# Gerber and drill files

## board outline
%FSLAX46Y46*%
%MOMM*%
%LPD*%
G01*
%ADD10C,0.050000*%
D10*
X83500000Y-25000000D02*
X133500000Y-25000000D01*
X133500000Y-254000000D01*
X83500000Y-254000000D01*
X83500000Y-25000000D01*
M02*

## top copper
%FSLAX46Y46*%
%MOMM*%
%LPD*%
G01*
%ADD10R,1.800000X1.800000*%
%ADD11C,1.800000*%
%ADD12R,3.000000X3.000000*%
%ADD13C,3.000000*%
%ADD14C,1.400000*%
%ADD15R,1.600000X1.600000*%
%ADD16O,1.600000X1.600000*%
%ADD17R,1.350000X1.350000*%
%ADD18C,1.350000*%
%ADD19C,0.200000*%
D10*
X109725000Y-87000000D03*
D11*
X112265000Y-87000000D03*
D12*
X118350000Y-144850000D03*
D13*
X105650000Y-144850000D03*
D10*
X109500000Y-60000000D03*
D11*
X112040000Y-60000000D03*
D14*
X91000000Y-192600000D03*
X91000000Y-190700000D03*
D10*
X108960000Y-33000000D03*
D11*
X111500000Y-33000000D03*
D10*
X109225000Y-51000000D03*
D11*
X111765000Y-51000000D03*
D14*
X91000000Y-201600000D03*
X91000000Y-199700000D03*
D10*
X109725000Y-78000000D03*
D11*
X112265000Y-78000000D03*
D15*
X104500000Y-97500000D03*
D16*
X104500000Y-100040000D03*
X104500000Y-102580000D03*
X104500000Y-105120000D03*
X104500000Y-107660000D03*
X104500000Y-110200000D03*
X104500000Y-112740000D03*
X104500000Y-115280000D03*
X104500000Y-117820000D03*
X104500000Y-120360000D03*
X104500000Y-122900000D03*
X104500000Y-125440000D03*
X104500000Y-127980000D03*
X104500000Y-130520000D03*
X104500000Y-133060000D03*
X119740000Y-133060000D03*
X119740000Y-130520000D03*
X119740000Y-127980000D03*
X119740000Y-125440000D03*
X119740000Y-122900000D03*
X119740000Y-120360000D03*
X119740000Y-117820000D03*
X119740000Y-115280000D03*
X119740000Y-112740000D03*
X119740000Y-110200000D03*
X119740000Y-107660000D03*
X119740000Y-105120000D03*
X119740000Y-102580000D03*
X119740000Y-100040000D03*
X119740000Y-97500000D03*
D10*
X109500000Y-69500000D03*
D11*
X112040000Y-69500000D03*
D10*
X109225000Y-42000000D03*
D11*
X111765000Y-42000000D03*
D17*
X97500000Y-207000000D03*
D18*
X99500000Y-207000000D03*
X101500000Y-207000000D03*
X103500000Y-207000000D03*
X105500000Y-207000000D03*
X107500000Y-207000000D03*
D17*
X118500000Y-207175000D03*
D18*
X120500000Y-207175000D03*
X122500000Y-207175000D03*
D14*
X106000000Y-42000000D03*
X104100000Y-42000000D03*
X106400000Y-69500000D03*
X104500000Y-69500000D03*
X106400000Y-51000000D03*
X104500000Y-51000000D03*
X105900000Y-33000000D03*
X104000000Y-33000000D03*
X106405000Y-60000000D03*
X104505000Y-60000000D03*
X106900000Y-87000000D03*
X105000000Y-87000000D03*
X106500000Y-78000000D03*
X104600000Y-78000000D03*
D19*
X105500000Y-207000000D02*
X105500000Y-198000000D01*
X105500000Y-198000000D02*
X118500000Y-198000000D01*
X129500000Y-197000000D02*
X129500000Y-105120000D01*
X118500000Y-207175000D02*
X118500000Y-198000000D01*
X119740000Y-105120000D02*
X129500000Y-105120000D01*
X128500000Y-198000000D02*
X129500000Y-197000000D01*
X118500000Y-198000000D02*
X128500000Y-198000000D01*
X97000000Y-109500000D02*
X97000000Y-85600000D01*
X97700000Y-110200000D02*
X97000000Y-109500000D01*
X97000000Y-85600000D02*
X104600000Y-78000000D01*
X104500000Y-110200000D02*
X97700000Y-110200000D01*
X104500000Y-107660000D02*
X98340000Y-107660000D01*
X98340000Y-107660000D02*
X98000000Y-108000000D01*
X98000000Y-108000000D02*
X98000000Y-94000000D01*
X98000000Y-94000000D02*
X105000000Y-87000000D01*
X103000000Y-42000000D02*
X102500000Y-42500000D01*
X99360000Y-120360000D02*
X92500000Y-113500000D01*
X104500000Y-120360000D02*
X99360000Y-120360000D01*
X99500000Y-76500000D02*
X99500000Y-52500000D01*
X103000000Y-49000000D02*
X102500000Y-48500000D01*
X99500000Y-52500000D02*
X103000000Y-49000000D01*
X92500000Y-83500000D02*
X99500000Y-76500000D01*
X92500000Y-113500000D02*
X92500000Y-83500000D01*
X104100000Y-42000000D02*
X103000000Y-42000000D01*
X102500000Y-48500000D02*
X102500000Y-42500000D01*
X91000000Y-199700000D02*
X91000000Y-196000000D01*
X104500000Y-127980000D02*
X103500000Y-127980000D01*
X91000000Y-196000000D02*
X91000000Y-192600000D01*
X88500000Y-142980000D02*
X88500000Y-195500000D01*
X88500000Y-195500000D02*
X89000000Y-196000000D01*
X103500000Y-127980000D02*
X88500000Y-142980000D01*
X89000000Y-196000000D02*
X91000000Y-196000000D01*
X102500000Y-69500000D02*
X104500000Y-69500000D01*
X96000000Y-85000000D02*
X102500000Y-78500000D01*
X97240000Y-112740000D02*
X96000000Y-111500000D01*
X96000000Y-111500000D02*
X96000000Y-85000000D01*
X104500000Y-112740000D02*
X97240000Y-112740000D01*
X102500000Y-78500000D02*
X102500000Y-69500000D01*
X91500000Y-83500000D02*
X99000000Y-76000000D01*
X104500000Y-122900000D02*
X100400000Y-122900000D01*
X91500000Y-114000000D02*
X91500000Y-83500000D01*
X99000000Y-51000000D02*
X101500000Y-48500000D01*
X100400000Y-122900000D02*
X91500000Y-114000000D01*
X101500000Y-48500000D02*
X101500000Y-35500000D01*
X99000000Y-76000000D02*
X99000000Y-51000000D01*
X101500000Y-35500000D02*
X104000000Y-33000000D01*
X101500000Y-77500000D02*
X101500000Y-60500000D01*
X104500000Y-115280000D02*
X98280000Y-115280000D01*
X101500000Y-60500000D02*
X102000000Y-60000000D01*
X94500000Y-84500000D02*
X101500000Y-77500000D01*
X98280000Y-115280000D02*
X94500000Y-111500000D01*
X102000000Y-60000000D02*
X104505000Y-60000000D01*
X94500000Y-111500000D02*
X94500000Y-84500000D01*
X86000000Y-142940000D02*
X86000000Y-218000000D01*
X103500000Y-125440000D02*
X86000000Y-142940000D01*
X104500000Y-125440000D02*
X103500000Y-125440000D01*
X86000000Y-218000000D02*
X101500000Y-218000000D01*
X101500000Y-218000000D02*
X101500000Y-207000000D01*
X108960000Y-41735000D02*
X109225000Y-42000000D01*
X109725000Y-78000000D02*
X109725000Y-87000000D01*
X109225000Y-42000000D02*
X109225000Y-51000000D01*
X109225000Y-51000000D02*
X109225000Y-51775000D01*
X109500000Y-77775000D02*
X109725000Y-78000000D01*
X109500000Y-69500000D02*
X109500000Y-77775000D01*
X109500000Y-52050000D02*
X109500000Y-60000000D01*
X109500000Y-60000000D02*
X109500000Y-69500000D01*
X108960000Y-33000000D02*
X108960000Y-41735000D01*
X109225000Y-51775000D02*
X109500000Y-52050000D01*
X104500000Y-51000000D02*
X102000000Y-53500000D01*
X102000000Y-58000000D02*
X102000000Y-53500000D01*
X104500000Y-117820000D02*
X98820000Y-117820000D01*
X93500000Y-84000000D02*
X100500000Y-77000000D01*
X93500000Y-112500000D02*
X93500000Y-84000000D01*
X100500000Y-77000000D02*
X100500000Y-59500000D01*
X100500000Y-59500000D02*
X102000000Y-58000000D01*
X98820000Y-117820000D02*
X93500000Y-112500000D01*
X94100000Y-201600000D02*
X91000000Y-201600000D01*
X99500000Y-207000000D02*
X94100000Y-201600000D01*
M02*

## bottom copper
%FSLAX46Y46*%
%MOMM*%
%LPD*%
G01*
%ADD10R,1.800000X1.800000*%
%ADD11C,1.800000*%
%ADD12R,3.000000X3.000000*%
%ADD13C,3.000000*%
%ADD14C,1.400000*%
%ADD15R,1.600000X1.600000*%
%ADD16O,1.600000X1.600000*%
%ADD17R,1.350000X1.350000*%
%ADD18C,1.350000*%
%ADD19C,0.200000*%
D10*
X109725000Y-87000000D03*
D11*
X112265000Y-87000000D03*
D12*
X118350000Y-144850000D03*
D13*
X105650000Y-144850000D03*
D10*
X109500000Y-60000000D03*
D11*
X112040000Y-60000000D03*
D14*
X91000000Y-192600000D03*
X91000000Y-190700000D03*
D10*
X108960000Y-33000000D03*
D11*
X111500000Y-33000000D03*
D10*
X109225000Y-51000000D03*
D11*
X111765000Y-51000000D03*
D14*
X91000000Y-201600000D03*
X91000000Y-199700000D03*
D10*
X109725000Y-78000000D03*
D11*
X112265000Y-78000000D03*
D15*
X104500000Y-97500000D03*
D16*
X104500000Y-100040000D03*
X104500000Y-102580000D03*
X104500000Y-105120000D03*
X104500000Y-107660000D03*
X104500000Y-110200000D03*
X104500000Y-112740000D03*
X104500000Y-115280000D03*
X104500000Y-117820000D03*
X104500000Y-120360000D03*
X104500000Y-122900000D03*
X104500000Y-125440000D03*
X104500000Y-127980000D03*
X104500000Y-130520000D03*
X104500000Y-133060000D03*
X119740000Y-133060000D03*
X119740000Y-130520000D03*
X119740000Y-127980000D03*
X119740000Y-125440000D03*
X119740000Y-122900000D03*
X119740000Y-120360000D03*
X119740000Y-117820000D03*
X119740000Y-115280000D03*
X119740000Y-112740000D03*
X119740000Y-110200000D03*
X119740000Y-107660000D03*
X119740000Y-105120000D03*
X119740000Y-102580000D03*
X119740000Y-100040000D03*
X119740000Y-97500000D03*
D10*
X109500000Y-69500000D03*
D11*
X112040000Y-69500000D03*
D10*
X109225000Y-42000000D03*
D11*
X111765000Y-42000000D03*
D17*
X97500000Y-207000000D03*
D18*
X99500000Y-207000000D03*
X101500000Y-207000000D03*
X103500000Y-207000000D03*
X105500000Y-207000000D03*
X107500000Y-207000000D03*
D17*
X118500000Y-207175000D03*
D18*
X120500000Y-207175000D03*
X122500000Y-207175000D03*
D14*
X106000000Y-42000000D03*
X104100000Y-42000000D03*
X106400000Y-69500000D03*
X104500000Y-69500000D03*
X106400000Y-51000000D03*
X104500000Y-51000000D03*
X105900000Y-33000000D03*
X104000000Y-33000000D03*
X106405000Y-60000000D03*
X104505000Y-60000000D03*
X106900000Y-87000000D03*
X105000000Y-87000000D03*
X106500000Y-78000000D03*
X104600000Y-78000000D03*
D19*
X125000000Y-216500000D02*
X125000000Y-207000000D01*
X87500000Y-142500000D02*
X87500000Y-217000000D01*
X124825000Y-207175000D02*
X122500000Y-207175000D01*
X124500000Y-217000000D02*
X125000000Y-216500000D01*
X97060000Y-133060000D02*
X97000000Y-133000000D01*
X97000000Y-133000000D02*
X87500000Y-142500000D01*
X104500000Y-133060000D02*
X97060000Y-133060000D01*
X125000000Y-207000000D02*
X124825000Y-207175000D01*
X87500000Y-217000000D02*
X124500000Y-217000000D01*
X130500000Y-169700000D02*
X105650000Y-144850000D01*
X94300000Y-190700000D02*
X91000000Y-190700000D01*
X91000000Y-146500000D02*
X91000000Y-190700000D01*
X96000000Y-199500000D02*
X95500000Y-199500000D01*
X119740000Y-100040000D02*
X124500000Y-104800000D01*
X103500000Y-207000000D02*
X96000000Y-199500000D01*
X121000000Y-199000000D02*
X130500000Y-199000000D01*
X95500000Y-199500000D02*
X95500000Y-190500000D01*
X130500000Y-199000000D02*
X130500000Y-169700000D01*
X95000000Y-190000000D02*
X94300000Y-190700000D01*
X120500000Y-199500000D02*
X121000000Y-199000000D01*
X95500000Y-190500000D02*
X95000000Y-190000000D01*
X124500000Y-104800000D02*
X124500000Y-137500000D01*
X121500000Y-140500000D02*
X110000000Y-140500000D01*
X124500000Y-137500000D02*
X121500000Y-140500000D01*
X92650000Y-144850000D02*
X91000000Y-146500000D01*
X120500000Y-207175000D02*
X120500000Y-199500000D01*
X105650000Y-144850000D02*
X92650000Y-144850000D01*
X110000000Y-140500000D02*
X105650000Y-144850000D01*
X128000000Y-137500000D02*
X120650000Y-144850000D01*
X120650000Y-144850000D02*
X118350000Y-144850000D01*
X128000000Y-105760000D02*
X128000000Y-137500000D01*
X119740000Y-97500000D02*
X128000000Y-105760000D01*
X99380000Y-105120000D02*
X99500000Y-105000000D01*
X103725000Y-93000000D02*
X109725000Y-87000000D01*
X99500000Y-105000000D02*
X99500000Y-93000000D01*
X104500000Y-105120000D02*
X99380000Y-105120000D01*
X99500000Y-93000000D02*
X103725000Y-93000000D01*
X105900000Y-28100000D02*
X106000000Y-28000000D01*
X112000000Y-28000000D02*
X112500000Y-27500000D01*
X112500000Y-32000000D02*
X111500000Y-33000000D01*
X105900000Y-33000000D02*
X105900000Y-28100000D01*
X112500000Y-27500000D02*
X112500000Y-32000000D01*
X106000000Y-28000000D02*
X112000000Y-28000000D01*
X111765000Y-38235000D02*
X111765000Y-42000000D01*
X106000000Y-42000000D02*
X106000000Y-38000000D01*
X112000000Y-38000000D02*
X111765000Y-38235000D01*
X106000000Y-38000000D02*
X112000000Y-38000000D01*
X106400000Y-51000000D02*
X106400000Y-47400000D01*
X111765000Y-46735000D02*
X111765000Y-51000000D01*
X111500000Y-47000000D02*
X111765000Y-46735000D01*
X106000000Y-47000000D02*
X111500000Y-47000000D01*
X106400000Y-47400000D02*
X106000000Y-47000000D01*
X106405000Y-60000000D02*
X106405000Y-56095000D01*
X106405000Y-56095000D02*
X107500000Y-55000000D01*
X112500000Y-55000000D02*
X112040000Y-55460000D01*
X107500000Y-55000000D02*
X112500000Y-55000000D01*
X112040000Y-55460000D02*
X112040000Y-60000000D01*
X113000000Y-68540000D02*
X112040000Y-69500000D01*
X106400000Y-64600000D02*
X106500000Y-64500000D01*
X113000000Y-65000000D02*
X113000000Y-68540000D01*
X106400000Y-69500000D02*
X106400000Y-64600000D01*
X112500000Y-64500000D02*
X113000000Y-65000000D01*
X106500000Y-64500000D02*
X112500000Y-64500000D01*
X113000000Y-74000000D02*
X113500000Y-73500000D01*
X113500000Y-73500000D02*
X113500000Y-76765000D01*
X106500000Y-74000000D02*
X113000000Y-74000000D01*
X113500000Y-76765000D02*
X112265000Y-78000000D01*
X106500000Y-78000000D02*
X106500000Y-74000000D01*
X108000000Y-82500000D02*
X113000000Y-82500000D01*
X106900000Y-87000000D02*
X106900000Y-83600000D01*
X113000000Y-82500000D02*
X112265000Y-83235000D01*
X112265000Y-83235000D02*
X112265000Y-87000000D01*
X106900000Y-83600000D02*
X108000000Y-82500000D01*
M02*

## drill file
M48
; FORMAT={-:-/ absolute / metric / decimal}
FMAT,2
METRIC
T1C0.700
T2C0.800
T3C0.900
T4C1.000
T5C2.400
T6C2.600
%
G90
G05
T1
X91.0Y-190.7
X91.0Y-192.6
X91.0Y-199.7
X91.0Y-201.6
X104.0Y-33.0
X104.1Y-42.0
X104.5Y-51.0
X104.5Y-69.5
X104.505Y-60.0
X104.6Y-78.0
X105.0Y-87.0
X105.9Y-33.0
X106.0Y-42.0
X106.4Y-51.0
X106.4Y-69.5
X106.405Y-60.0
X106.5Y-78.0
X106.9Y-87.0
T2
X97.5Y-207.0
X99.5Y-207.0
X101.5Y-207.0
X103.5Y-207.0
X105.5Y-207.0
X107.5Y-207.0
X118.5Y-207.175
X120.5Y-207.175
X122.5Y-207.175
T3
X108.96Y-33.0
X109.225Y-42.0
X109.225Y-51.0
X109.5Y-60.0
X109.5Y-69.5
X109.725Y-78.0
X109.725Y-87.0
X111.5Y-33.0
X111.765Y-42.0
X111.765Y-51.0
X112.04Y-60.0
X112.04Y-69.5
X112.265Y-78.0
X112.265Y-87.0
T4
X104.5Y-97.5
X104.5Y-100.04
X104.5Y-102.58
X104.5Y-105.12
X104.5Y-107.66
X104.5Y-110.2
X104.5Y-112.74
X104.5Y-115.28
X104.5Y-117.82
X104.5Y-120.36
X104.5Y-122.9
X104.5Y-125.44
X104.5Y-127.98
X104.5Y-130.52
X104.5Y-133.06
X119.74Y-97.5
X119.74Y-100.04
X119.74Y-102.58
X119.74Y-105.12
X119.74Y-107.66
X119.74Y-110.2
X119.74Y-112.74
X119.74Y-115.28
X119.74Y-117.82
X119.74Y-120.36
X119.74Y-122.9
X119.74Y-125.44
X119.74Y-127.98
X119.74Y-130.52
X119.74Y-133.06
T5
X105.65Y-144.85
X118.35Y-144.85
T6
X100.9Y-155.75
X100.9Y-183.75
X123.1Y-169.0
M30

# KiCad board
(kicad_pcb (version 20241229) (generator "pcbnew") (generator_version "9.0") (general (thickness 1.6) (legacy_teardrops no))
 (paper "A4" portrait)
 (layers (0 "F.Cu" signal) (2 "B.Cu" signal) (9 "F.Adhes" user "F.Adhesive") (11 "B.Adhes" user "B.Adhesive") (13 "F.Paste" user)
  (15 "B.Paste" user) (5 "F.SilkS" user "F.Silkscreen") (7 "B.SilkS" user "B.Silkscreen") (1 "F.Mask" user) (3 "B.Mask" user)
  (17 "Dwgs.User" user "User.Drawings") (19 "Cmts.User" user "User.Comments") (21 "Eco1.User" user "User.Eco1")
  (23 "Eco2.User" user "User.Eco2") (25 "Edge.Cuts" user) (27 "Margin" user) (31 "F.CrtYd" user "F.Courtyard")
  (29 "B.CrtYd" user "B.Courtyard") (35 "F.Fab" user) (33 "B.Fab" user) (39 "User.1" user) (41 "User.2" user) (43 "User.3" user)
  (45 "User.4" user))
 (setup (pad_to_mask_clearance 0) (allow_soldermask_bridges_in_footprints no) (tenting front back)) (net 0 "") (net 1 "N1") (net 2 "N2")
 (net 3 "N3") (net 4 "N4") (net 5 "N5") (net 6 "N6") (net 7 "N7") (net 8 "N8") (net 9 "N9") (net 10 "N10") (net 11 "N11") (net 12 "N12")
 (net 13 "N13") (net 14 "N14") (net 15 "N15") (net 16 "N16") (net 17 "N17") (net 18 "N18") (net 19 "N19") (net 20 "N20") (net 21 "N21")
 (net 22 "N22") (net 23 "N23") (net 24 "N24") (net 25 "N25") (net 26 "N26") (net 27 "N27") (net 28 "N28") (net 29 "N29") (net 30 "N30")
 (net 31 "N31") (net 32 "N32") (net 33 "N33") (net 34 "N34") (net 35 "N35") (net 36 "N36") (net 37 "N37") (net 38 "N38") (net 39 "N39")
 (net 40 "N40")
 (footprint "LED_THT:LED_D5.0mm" (layer "F.Cu") (at 109.725 87)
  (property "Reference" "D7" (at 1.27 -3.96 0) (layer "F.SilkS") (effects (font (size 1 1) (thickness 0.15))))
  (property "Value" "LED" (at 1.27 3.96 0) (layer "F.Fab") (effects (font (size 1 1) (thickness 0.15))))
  (pad "1" thru_hole rect (at 0 0) (size 1.8 1.8) (drill 0.9) (layers "*.Cu" "*.Mask") (remove_unused_layers no) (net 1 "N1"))
  (pad "2" thru_hole circle (at 2.54 0) (size 1.8 1.8) (drill 0.9) (layers "*.Cu" "*.Mask") (remove_unused_layers no) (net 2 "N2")))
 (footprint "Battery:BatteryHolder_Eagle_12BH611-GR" (layer "F.Cu") (at 118.35 144.85 90)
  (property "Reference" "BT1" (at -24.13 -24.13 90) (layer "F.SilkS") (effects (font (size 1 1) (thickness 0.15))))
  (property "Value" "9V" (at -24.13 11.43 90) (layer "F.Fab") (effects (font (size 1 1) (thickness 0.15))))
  (pad "" np_thru_hole circle (at -38.9 -17.45 90) (size 2.6 2.6) (drill 2.6) (layers "*.Cu" "*.Mask"))
  (pad "" np_thru_hole circle (at -24.15 4.75 90) (size 2.6 2.6) (drill 2.6) (layers "*.Cu" "*.Mask"))
  (pad "" np_thru_hole circle (at -10.9 -17.45 90) (size 2.6 2.6) (drill 2.6) (layers "*.Cu" "*.Mask"))
  (pad "1" thru_hole rect (at 0 0 90) (size 3 3) (drill 2.4) (layers "*.Cu" "*.Mask") (remove_unused_layers no) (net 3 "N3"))
  (pad "2" thru_hole circle (at 0 -12.7 90) (size 3 3) (drill 2.4) (layers "*.Cu" "*.Mask") (remove_unused_layers no) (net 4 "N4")))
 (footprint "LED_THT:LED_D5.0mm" (layer "F.Cu") (at 109.5 60)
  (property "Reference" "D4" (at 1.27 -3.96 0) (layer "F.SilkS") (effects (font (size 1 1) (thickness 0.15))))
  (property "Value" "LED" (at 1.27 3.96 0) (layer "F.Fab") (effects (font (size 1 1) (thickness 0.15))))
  (pad "1" thru_hole rect (at 0 0) (size 1.8 1.8) (drill 0.9) (layers "*.Cu" "*.Mask") (remove_unused_layers no) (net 1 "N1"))
  (pad "2" thru_hole circle (at 2.54 0) (size 1.8 1.8) (drill 0.9) (layers "*.Cu" "*.Mask") (remove_unused_layers no) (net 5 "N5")))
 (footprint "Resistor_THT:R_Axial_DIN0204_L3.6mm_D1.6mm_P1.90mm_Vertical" (layer "F.Cu") (at 91 192.6 90)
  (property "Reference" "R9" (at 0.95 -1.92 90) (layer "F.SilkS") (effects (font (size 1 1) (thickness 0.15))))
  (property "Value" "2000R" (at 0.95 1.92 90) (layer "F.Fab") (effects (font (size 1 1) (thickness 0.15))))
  (pad "1" thru_hole circle (at 0 0 90) (size 1.4 1.4) (drill 0.7) (layers "*.Cu" "*.Mask") (remove_unused_layers no) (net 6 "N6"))
  (pad "2" thru_hole circle (at 1.9 0 90) (size 1.4 1.4) (drill 0.7) (layers "*.Cu" "*.Mask") (remove_unused_layers no) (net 4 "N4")))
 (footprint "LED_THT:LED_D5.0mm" (layer "F.Cu") (at 108.96 33)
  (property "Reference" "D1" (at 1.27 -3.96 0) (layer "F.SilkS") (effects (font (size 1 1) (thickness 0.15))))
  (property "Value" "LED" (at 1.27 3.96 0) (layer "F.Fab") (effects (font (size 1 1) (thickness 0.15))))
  (pad "1" thru_hole rect (at 0 0) (size 1.8 1.8) (drill 0.9) (layers "*.Cu" "*.Mask") (remove_unused_layers no) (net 1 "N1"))
  (pad "2" thru_hole circle (at 2.54 0) (size 1.8 1.8) (drill 0.9) (layers "*.Cu" "*.Mask") (remove_unused_layers no) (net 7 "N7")))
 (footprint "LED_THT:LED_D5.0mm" (layer "F.Cu") (at 109.225 51)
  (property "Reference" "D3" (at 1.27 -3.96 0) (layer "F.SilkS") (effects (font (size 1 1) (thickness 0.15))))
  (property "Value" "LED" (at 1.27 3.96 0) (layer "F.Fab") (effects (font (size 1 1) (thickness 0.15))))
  (pad "1" thru_hole rect (at 0 0) (size 1.8 1.8) (drill 0.9) (layers "*.Cu" "*.Mask") (remove_unused_layers no) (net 1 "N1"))
  (pad "2" thru_hole circle (at 2.54 0) (size 1.8 1.8) (drill 0.9) (layers "*.Cu" "*.Mask") (remove_unused_layers no) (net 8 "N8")))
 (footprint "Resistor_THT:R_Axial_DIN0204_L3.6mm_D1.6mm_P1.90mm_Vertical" (layer "F.Cu") (at 91 201.6 90)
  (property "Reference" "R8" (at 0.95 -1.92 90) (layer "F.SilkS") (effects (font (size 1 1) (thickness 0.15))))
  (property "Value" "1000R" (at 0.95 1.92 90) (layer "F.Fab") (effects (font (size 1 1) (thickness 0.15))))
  (pad "1" thru_hole circle (at 0 0 90) (size 1.4 1.4) (drill 0.7) (layers "*.Cu" "*.Mask") (remove_unused_layers no) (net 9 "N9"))
  (pad "2" thru_hole circle (at 1.9 0 90) (size 1.4 1.4) (drill 0.7) (layers "*.Cu" "*.Mask") (remove_unused_layers no) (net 6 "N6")))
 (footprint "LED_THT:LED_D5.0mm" (layer "F.Cu") (at 109.725 78)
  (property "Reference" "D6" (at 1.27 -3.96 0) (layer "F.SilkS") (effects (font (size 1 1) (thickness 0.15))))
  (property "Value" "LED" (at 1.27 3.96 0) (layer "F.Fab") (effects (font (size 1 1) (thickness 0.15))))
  (pad "1" thru_hole rect (at 0 0) (size 1.8 1.8) (drill 0.9) (layers "*.Cu" "*.Mask") (remove_unused_layers no) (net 1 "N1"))
  (pad "2" thru_hole circle (at 2.54 0) (size 1.8 1.8) (drill 0.9) (layers "*.Cu" "*.Mask") (remove_unused_layers no) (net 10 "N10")))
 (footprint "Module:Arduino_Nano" (layer "F.Cu") (at 104.5 97.5)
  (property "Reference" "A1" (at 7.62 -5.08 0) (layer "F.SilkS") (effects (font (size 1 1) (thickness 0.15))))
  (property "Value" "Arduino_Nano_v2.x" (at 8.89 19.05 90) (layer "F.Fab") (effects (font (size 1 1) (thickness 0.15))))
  (pad "1" thru_hole rect (at 0 0) (size 1.6 1.6) (drill 1) (layers "*.Cu" "*.Mask") (remove_unused_layers no) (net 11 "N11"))
  (pad "2" thru_hole oval (at 0 2.54) (size 1.6 1.6) (drill 1) (layers "*.Cu" "*.Mask") (remove_unused_layers no) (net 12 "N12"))
  (pad "3" thru_hole oval (at 0 5.08) (size 1.6 1.6) (drill 1) (layers "*.Cu" "*.Mask") (remove_unused_layers no) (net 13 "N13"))
  (pad "4" thru_hole oval (at 0 7.62) (size 1.6 1.6) (drill 1) (layers "*.Cu" "*.Mask") (remove_unused_layers no) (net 1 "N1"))
  (pad "5" thru_hole oval (at 0 10.16) (size 1.6 1.6) (drill 1) (layers "*.Cu" "*.Mask") (remove_unused_layers no) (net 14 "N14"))
  (pad "6" thru_hole oval (at 0 12.7) (size 1.6 1.6) (drill 1) (layers "*.Cu" "*.Mask") (remove_unused_layers no) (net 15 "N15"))
  (pad "7" thru_hole oval (at 0 15.24) (size 1.6 1.6) (drill 1) (layers "*.Cu" "*.Mask") (remove_unused_layers no) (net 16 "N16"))
  (pad "8" thru_hole oval (at 0 17.78) (size 1.6 1.6) (drill 1) (layers "*.Cu" "*.Mask") (remove_unused_layers no) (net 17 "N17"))
  (pad "9" thru_hole oval (at 0 20.32) (size 1.6 1.6) (drill 1) (layers "*.Cu" "*.Mask") (remove_unused_layers no) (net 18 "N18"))
  (pad "10" thru_hole oval (at 0 22.86) (size 1.6 1.6) (drill 1) (layers "*.Cu" "*.Mask") (remove_unused_layers no) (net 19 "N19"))
  (pad "11" thru_hole oval (at 0 25.4) (size 1.6 1.6) (drill 1) (layers "*.Cu" "*.Mask") (remove_unused_layers no) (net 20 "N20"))
  (pad "12" thru_hole oval (at 0 27.94) (size 1.6 1.6) (drill 1) (layers "*.Cu" "*.Mask") (remove_unused_layers no) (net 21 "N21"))
  (pad "13" thru_hole oval (at 0 30.48) (size 1.6 1.6) (drill 1) (layers "*.Cu" "*.Mask") (remove_unused_layers no) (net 6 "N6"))
  (pad "14" thru_hole oval (at 0 33.02) (size 1.6 1.6) (drill 1) (layers "*.Cu" "*.Mask") (remove_unused_layers no) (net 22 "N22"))
  (pad "15" thru_hole oval (at 0 35.56) (size 1.6 1.6) (drill 1) (layers "*.Cu" "*.Mask") (remove_unused_layers no) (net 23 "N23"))
  (pad "16" thru_hole oval (at 15.24 35.56) (size 1.6 1.6) (drill 1) (layers "*.Cu" "*.Mask") (remove_unused_layers no) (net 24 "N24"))
  (pad "17" thru_hole oval (at 15.24 33.02) (size 1.6 1.6) (drill 1) (layers "*.Cu" "*.Mask") (remove_unused_layers no) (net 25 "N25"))
  (pad "18" thru_hole oval (at 15.24 30.48) (size 1.6 1.6) (drill 1) (layers "*.Cu" "*.Mask") (remove_unused_layers no) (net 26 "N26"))
  (pad "19" thru_hole oval (at 15.24 27.94) (size 1.6 1.6) (drill 1) (layers "*.Cu" "*.Mask") (remove_unused_layers no) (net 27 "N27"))
  (pad "20" thru_hole oval (at 15.24 25.4) (size 1.6 1.6) (drill 1) (layers "*.Cu" "*.Mask") (remove_unused_layers no) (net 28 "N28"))
  (pad "21" thru_hole oval (at 15.24 22.86) (size 1.6 1.6) (drill 1) (layers "*.Cu" "*.Mask") (remove_unused_layers no) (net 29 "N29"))
  (pad "22" thru_hole oval (at 15.24 20.32) (size 1.6 1.6) (drill 1) (layers "*.Cu" "*.Mask") (remove_unused_layers no) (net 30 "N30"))
  (pad "23" thru_hole oval (at 15.24 17.78) (size 1.6 1.6) (drill 1) (layers "*.Cu" "*.Mask") (remove_unused_layers no) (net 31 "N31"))
  (pad "24" thru_hole oval (at 15.24 15.24) (size 1.6 1.6) (drill 1) (layers "*.Cu" "*.Mask") (remove_unused_layers no) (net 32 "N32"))
  (pad "25" thru_hole oval (at 15.24 12.7) (size 1.6 1.6) (drill 1) (layers "*.Cu" "*.Mask") (remove_unused_layers no) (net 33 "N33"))
  (pad "26" thru_hole oval (at 15.24 10.16) (size 1.6 1.6) (drill 1) (layers "*.Cu" "*.Mask") (remove_unused_layers no) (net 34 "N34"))
  (pad "27" thru_hole oval (at 15.24 7.62) (size 1.6 1.6) (drill 1) (layers "*.Cu" "*.Mask") (remove_unused_layers no) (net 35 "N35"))
  (pad "28" thru_hole oval (at 15.24 5.08) (size 1.6 1.6) (drill 1) (layers "*.Cu" "*.Mask") (remove_unused_layers no) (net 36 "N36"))
  (pad "29" thru_hole oval (at 15.24 2.54) (size 1.6 1.6) (drill 1) (layers "*.Cu" "*.Mask") (remove_unused_layers no) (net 4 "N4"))
  (pad "30" thru_hole oval (at 15.24 0) (size 1.6 1.6) (drill 1) (layers "*.Cu" "*.Mask") (remove_unused_layers no) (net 3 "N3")))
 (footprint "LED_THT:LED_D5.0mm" (layer "F.Cu") (at 109.5 69.5)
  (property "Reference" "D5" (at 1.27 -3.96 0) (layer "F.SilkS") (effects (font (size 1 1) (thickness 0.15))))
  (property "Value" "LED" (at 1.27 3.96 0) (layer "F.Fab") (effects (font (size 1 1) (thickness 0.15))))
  (pad "1" thru_hole rect (at 0 0) (size 1.8 1.8) (drill 0.9) (layers "*.Cu" "*.Mask") (remove_unused_layers no) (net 1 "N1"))
  (pad "2" thru_hole circle (at 2.54 0) (size 1.8 1.8) (drill 0.9) (layers "*.Cu" "*.Mask") (remove_unused_layers no) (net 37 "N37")))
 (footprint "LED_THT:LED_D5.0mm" (layer "F.Cu") (at 109.225 42)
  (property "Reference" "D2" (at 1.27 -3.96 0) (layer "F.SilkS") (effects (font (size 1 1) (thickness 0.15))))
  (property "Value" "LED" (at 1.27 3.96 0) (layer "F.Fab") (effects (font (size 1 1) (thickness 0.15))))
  (pad "1" thru_hole rect (at 0 0) (size 1.8 1.8) (drill 0.9) (layers "*.Cu" "*.Mask") (remove_unused_layers no) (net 1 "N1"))
  (pad "2" thru_hole circle (at 2.54 0) (size 1.8 1.8) (drill 0.9) (layers "*.Cu" "*.Mask") (remove_unused_layers no) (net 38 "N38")))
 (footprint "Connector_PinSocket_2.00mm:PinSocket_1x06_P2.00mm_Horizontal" (layer "F.Cu") (at 97.5 207 90)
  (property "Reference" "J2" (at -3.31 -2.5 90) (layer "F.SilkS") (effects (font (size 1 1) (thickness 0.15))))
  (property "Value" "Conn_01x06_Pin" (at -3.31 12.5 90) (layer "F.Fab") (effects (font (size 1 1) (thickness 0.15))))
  (pad "1" thru_hole rect (at 0 0 90) (size 1.35 1.35) (drill 0.8) (layers "*.Cu" "*.Mask") (remove_unused_layers no) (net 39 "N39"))
  (pad "2" thru_hole circle (at 0 2 90) (size 1.35 1.35) (drill 0.8) (layers "*.Cu" "*.Mask") (remove_unused_layers no) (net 9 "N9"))
  (pad "3" thru_hole circle (at 0 4 90) (size 1.35 1.35) (drill 0.8) (layers "*.Cu" "*.Mask") (remove_unused_layers no) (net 21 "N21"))
  (pad "4" thru_hole circle (at 0 6 90) (size 1.35 1.35) (drill 0.8) (layers "*.Cu" "*.Mask") (remove_unused_layers no) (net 4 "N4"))
  (pad "5" thru_hole circle (at 0 8 90) (size 1.35 1.35) (drill 0.8) (layers "*.Cu" "*.Mask") (remove_unused_layers no) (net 35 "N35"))
  (pad "6" thru_hole circle (at 0 10 90) (size 1.35 1.35) (drill 0.8) (layers "*.Cu" "*.Mask") (remove_unused_layers no) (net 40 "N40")))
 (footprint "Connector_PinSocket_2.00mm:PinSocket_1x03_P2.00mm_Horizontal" (layer "F.Cu") (at 118.5 207.175 90)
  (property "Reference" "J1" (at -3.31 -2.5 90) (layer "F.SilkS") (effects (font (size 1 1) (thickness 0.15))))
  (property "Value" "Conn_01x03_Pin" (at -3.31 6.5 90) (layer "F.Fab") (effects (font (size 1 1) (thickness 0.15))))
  (pad "1" thru_hole rect (at 0 0 90) (size 1.35 1.35) (drill 0.8) (layers "*.Cu" "*.Mask") (remove_unused_layers no) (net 35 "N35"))
  (pad "2" thru_hole circle (at 0 2 90) (size 1.35 1.35) (drill 0.8) (layers "*.Cu" "*.Mask") (remove_unused_layers no) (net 4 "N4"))
  (pad "3" thru_hole circle (at 0 4 90) (size 1.35 1.35) (drill 0.8) (layers "*.Cu" "*.Mask") (remove_unused_layers no) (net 23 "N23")))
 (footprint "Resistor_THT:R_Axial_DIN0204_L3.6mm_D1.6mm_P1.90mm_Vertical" (layer "B.Cu") (at 106 42 180)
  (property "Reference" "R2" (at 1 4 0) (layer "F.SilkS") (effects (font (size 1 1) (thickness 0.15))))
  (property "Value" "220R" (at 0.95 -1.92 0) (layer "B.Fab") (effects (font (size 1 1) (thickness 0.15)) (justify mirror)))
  (pad "1" thru_hole circle (at 0 0 180) (size 1.4 1.4) (drill 0.7) (layers "*.Cu" "*.Mask") (remove_unused_layers no) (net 38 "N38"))
  (pad "2" thru_hole circle (at 1.9 0 180) (size 1.4 1.4) (drill 0.7) (layers "*.Cu" "*.Mask") (remove_unused_layers no) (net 19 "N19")))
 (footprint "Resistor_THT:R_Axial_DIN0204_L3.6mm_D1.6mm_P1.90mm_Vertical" (layer "B.Cu") (at 106.4 69.5 180)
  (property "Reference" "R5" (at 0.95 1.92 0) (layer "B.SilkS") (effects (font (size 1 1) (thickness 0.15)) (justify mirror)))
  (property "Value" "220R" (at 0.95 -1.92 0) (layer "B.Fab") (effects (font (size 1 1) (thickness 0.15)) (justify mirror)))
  (pad "1" thru_hole circle (at 0 0 180) (size 1.4 1.4) (drill 0.7) (layers "*.Cu" "*.Mask") (remove_unused_layers no) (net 37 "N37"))
  (pad "2" thru_hole circle (at 1.9 0 180) (size 1.4 1.4) (drill 0.7) (layers "*.Cu" "*.Mask") (remove_unused_layers no) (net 16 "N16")))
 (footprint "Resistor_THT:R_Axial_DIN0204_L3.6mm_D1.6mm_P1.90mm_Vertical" (layer "B.Cu") (at 106.4 51 180)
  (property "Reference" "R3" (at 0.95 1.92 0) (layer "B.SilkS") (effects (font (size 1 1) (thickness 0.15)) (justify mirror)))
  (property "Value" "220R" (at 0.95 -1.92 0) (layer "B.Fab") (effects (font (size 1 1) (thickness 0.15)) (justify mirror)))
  (pad "1" thru_hole circle (at 0 0 180) (size 1.4 1.4) (drill 0.7) (layers "*.Cu" "*.Mask") (remove_unused_layers no) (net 8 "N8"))
  (pad "2" thru_hole circle (at 1.9 0 180) (size 1.4 1.4) (drill 0.7) (layers "*.Cu" "*.Mask") (remove_unused_layers no) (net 18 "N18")))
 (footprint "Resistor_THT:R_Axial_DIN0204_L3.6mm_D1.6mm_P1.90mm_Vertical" (layer "B.Cu") (at 105.9 33 180)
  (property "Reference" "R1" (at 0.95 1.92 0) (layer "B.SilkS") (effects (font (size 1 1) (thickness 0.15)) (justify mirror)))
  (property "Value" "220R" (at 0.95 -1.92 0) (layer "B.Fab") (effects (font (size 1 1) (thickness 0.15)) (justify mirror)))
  (pad "1" thru_hole circle (at 0 0 180) (size 1.4 1.4) (drill 0.7) (layers "*.Cu" "*.Mask") (remove_unused_layers no) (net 7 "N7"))
  (pad "2" thru_hole circle (at 1.9 0 180) (size 1.4 1.4) (drill 0.7) (layers "*.Cu" "*.Mask") (remove_unused_layers no) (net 20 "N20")))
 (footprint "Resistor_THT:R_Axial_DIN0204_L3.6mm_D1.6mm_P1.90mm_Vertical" (layer "B.Cu") (at 106.405 60 180)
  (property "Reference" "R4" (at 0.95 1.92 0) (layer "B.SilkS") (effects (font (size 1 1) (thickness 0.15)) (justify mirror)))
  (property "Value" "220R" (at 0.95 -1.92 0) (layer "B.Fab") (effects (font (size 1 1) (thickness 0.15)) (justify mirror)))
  (pad "1" thru_hole circle (at 0 0 180) (size 1.4 1.4) (drill 0.7) (layers "*.Cu" "*.Mask") (remove_unused_layers no) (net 5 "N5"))
  (pad "2" thru_hole circle (at 1.9 0 180) (size 1.4 1.4) (drill 0.7) (layers "*.Cu" "*.Mask") (remove_unused_layers no) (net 17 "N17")))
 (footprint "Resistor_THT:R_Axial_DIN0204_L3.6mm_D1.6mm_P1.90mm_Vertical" (layer "B.Cu") (at 106.9 87 180)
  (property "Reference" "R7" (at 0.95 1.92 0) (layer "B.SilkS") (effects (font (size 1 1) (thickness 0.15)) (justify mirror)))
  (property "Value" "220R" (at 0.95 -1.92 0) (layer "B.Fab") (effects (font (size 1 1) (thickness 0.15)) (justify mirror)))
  (pad "1" thru_hole circle (at 0 0 180) (size 1.4 1.4) (drill 0.7) (layers "*.Cu" "*.Mask") (remove_unused_layers no) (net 2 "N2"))
  (pad "2" thru_hole circle (at 1.9 0 180) (size 1.4 1.4) (drill 0.7) (layers "*.Cu" "*.Mask") (remove_unused_layers no) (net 14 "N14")))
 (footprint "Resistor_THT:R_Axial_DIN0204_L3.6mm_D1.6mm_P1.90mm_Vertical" (layer "B.Cu") (at 106.5 78 180)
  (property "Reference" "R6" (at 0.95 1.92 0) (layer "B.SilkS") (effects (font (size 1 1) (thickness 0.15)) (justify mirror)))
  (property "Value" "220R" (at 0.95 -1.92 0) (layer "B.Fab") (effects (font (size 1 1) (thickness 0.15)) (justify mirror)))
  (pad "1" thru_hole circle (at 0 0 180) (size 1.4 1.4) (drill 0.7) (layers "*.Cu" "*.Mask") (remove_unused_layers no) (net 10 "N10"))
  (pad "2" thru_hole circle (at 1.9 0 180) (size 1.4 1.4) (drill 0.7) (layers "*.Cu" "*.Mask") (remove_unused_layers no) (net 15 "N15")))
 (gr_rect (start 83.5 25) (end 133.5 254) (stroke (width 0.05) (type default)) (fill no) (layer "Edge.Cuts"))
 (segment (start 125 216.5) (end 125 207) (width 0.2) (layer "B.Cu") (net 23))
 (segment (start 87.5 142.5) (end 87.5 217) (width 0.2) (layer "B.Cu") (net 23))
 (segment (start 124.825 207.175) (end 122.5 207.175) (width 0.2) (layer "B.Cu") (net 23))
 (segment (start 124.5 217) (end 125 216.5) (width 0.2) (layer "B.Cu") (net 23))
 (segment (start 97.06 133.06) (end 97 133) (width 0.2) (layer "B.Cu") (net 23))
 (segment (start 97 133) (end 87.5 142.5) (width 0.2) (layer "B.Cu") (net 23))
 (segment (start 104.5 133.06) (end 97.06 133.06) (width 0.2) (layer "B.Cu") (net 23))
 (segment (start 125 207) (end 124.825 207.175) (width 0.2) (layer "B.Cu") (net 23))
 (segment (start 87.5 217) (end 124.5 217) (width 0.2) (layer "B.Cu") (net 23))
 (segment (start 130.5 169.7) (end 105.65 144.85) (width 0.2) (layer "B.Cu") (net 4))
 (segment (start 94.3 190.7) (end 91 190.7) (width 0.2) (layer "B.Cu") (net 4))
 (segment (start 91 146.5) (end 91 190.7) (width 0.2) (layer "B.Cu") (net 4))
 (segment (start 96 199.5) (end 95.5 199.5) (width 0.2) (layer "B.Cu") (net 4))
 (segment (start 119.74 100.04) (end 124.5 104.8) (width 0.2) (layer "B.Cu") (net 4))
 (segment (start 103.5 207) (end 96 199.5) (width 0.2) (layer "B.Cu") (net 4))
 (segment (start 121 199) (end 130.5 199) (width 0.2) (layer "B.Cu") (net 4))
 (segment (start 95.5 199.5) (end 95.5 190.5) (width 0.2) (layer "B.Cu") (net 4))
 (segment (start 130.5 199) (end 130.5 169.7) (width 0.2) (layer "B.Cu") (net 4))
 (segment (start 95 190) (end 94.3 190.7) (width 0.2) (layer "B.Cu") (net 4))
 (segment (start 120.5 199.5) (end 121 199) (width 0.2) (layer "B.Cu") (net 4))
 (segment (start 95.5 190.5) (end 95 190) (width 0.2) (layer "B.Cu") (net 4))
 (segment (start 124.5 104.8) (end 124.5 137.5) (width 0.2) (layer "B.Cu") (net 4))
 (segment (start 121.5 140.5) (end 110 140.5) (width 0.2) (layer "B.Cu") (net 4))
 (segment (start 124.5 137.5) (end 121.5 140.5) (width 0.2) (layer "B.Cu") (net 4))
 (segment (start 92.65 144.85) (end 91 146.5) (width 0.2) (layer "B.Cu") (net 4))
 (segment (start 120.5 207.175) (end 120.5 199.5) (width 0.2) (layer "B.Cu") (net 4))
 (segment (start 105.65 144.85) (end 92.65 144.85) (width 0.2) (layer "B.Cu") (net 4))
 (segment (start 110 140.5) (end 105.65 144.85) (width 0.2) (layer "B.Cu") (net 4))
 (segment (start 105.5 207) (end 105.5 198) (width 0.2) (layer "F.Cu") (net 35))
 (segment (start 105.5 198) (end 118.5 198) (width 0.2) (layer "F.Cu") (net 35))
 (segment (start 129.5 197) (end 129.5 105.12) (width 0.2) (layer "F.Cu") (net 35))
 (segment (start 118.5 207.175) (end 118.5 198) (width 0.2) (layer "F.Cu") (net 35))
 (segment (start 119.74 105.12) (end 129.5 105.12) (width 0.2) (layer "F.Cu") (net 35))
 (segment (start 128.5 198) (end 129.5 197) (width 0.2) (layer "F.Cu") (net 35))
 (segment (start 118.5 198) (end 128.5 198) (width 0.2) (layer "F.Cu") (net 35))
 (segment (start 97 109.5) (end 97 85.6) (width 0.2) (layer "F.Cu") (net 15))
 (segment (start 97.7 110.2) (end 97 109.5) (width 0.2) (layer "F.Cu") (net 15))
 (segment (start 97 85.6) (end 104.6 78) (width 0.2) (layer "F.Cu") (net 15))
 (segment (start 104.5 110.2) (end 97.7 110.2) (width 0.2) (layer "F.Cu") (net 15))
 (segment (start 104.5 107.66) (end 98.34 107.66) (width 0.2) (layer "F.Cu") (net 14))
 (segment (start 98.34 107.66) (end 98 108) (width 0.2) (layer "F.Cu") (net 14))
 (segment (start 98 108) (end 98 94) (width 0.2) (layer "F.Cu") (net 14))
 (segment (start 98 94) (end 105 87) (width 0.2) (layer "F.Cu") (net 14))
 (segment (start 128 137.5) (end 120.65 144.85) (width 0.2) (layer "B.Cu") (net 3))
 (segment (start 120.65 144.85) (end 118.35 144.85) (width 0.2) (layer "B.Cu") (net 3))
 (segment (start 128 105.76) (end 128 137.5) (width 0.2) (layer "B.Cu") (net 3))
 (segment (start 119.74 97.5) (end 128 105.76) (width 0.2) (layer "B.Cu") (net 3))
 (segment (start 103 42) (end 102.5 42.5) (width 0.2) (layer "F.Cu") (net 19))
 (segment (start 99.36 120.36) (end 92.5 113.5) (width 0.2) (layer "F.Cu") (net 19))
 (segment (start 104.5 120.36) (end 99.36 120.36) (width 0.2) (layer "F.Cu") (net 19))
 (segment (start 99.5 76.5) (end 99.5 52.5) (width 0.2) (layer "F.Cu") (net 19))
 (segment (start 103 49) (end 102.5 48.5) (width 0.2) (layer "F.Cu") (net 19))
 (segment (start 99.5 52.5) (end 103 49) (width 0.2) (layer "F.Cu") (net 19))
 (segment (start 92.5 83.5) (end 99.5 76.5) (width 0.2) (layer "F.Cu") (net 19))
 (segment (start 92.5 113.5) (end 92.5 83.5) (width 0.2) (layer "F.Cu") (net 19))
 (segment (start 104.1 42) (end 103 42) (width 0.2) (layer "F.Cu") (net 19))
 (segment (start 102.5 48.5) (end 102.5 42.5) (width 0.2) (layer "F.Cu") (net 19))
 (segment (start 91 199.7) (end 91 196) (width 0.2) (layer "F.Cu") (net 6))
 (segment (start 104.5 127.98) (end 103.5 127.98) (width 0.2) (layer "F.Cu") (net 6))
 (segment (start 91 196) (end 91 192.6) (width 0.2) (layer "F.Cu") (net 6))
 (segment (start 88.5 142.98) (end 88.5 195.5) (width 0.2) (layer "F.Cu") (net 6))
 (segment (start 88.5 195.5) (end 89 196) (width 0.2) (layer "F.Cu") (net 6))
 (segment (start 103.5 127.98) (end 88.5 142.98) (width 0.2) (layer "F.Cu") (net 6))
 (segment (start 89 196) (end 91 196) (width 0.2) (layer "F.Cu") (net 6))
 (segment (start 102.5 69.5) (end 104.5 69.5) (width 0.2) (layer "F.Cu") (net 16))
 (segment (start 96 85) (end 102.5 78.5) (width 0.2) (layer "F.Cu") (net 16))
 (segment (start 97.24 112.74) (end 96 111.5) (width 0.2) (layer "F.Cu") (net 16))
 (segment (start 96 111.5) (end 96 85) (width 0.2) (layer "F.Cu") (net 16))
 (segment (start 104.5 112.74) (end 97.24 112.74) (width 0.2) (layer "F.Cu") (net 16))
 (segment (start 102.5 78.5) (end 102.5 69.5) (width 0.2) (layer "F.Cu") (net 16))
 (segment (start 91.5 83.5) (end 99 76) (width 0.2) (layer "F.Cu") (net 20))
 (segment (start 104.5 122.9) (end 100.4 122.9) (width 0.2) (layer "F.Cu") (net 20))
 (segment (start 91.5 114) (end 91.5 83.5) (width 0.2) (layer "F.Cu") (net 20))
 (segment (start 99 51) (end 101.5 48.5) (width 0.2) (layer "F.Cu") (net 20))
 (segment (start 100.4 122.9) (end 91.5 114) (width 0.2) (layer "F.Cu") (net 20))
 (segment (start 101.5 48.5) (end 101.5 35.5) (width 0.2) (layer "F.Cu") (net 20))
 (segment (start 99 76) (end 99 51) (width 0.2) (layer "F.Cu") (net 20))
 (segment (start 101.5 35.5) (end 104 33) (width 0.2) (layer "F.Cu") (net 20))
 (segment (start 101.5 77.5) (end 101.5 60.5) (width 0.2) (layer "F.Cu") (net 17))
 (segment (start 104.5 115.28) (end 98.28 115.28) (width 0.2) (layer "F.Cu") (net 17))
 (segment (start 101.5 60.5) (end 102 60) (width 0.2) (layer "F.Cu") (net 17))
 (segment (start 94.5 84.5) (end 101.5 77.5) (width 0.2) (layer "F.Cu") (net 17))
 (segment (start 98.28 115.28) (end 94.5 111.5) (width 0.2) (layer "F.Cu") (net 17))
 (segment (start 102 60) (end 104.505 60) (width 0.2) (layer "F.Cu") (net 17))
 (segment (start 94.5 111.5) (end 94.5 84.5) (width 0.2) (layer "F.Cu") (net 17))
 (segment (start 86 142.94) (end 86 218) (width 0.2) (layer "F.Cu") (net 21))
 (segment (start 103.5 125.44) (end 86 142.94) (width 0.2) (layer "F.Cu") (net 21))
 (segment (start 104.5 125.44) (end 103.5 125.44) (width 0.2) (layer "F.Cu") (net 21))
 (segment (start 86 218) (end 101.5 218) (width 0.2) (layer "F.Cu") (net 21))
 (segment (start 101.5 218) (end 101.5 207) (width 0.2) (layer "F.Cu") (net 21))
 (segment (start 108.96 41.735) (end 109.225 42) (width 0.2) (layer "F.Cu") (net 1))
 (segment (start 109.725 78) (end 109.725 87) (width 0.2) (layer "F.Cu") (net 1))
 (segment (start 109.225 42) (end 109.225 51) (width 0.2) (layer "F.Cu") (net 1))
 (segment (start 109.225 51) (end 109.225 51.775) (width 0.2) (layer "F.Cu") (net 1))
 (segment (start 109.5 77.775) (end 109.725 78) (width 0.2) (layer "F.Cu") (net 1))
 (segment (start 109.5 69.5) (end 109.5 77.775) (width 0.2) (layer "F.Cu") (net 1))
 (segment (start 109.5 52.05) (end 109.5 60) (width 0.2) (layer "F.Cu") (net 1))
 (segment (start 109.5 60) (end 109.5 69.5) (width 0.2) (layer "F.Cu") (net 1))
 (segment (start 108.96 33) (end 108.96 41.735) (width 0.2) (layer "F.Cu") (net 1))
 (segment (start 109.225 51.775) (end 109.5 52.05) (width 0.2) (layer "F.Cu") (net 1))
 (segment (start 99.38 105.12) (end 99.5 105) (width 0.2) (layer "B.Cu") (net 1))
 (segment (start 103.725 93) (end 109.725 87) (width 0.2) (layer "B.Cu") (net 1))
 (segment (start 99.5 105) (end 99.5 93) (width 0.2) (layer "B.Cu") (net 1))
 (segment (start 104.5 105.12) (end 99.38 105.12) (width 0.2) (layer "B.Cu") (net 1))
 (segment (start 99.5 93) (end 103.725 93) (width 0.2) (layer "B.Cu") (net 1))
 (segment (start 104.5 51) (end 102 53.5) (width 0.2) (layer "F.Cu") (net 18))
 (segment (start 102 58) (end 102 53.5) (width 0.2) (layer "F.Cu") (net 18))
 (segment (start 104.5 117.82) (end 98.82 117.82) (width 0.2) (layer "F.Cu") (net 18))
 (segment (start 93.5 84) (end 100.5 77) (width 0.2) (layer "F.Cu") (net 18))
 (segment (start 93.5 112.5) (end 93.5 84) (width 0.2) (layer "F.Cu") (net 18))
 (segment (start 100.5 77) (end 100.5 59.5) (width 0.2) (layer "F.Cu") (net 18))
 (segment (start 100.5 59.5) (end 102 58) (width 0.2) (layer "F.Cu") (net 18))
 (segment (start 98.82 117.82) (end 93.5 112.5) (width 0.2) (layer "F.Cu") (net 18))
 (segment (start 105.9 28.1) (end 106 28) (width 0.2) (layer "B.Cu") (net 7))
 (segment (start 112 28) (end 112.5 27.5) (width 0.2) (layer "B.Cu") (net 7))
 (segment (start 112.5 32) (end 111.5 33) (width 0.2) (layer "B.Cu") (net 7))
 (segment (start 105.9 33) (end 105.9 28.1) (width 0.2) (layer "B.Cu") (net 7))
 (segment (start 112.5 27.5) (end 112.5 32) (width 0.2) (layer "B.Cu") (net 7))
 (segment (start 106 28) (end 112 28) (width 0.2) (layer "B.Cu") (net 7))
 (segment (start 111.765 38.235) (end 111.765 42) (width 0.2) (layer "B.Cu") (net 38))
 (segment (start 106 42) (end 106 38) (width 0.2) (layer "B.Cu") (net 38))
 (segment (start 112 38) (end 111.765 38.235) (width 0.2) (layer "B.Cu") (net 38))
 (segment (start 106 38) (end 112 38) (width 0.2) (layer "B.Cu") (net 38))
 (segment (start 106.4 51) (end 106.4 47.4) (width 0.2) (layer "B.Cu") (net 8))
 (segment (start 111.765 46.735) (end 111.765 51) (width 0.2) (layer "B.Cu") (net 8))
 (segment (start 111.5 47) (end 111.765 46.735) (width 0.2) (layer "B.Cu") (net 8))
 (segment (start 106 47) (end 111.5 47) (width 0.2) (layer "B.Cu") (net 8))
 (segment (start 106.4 47.4) (end 106 47) (width 0.2) (layer "B.Cu") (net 8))
 (segment (start 106.405 60) (end 106.405 56.095) (width 0.2) (layer "B.Cu") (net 5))
 (segment (start 106.405 56.095) (end 107.5 55) (width 0.2) (layer "B.Cu") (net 5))
 (segment (start 112.5 55) (end 112.04 55.46) (width 0.2) (layer "B.Cu") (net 5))
 (segment (start 107.5 55) (end 112.5 55) (width 0.2) (layer "B.Cu") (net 5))
 (segment (start 112.04 55.46) (end 112.04 60) (width 0.2) (layer "B.Cu") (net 5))
 (segment (start 113 68.54) (end 112.04 69.5) (width 0.2) (layer "B.Cu") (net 37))
 (segment (start 106.4 64.6) (end 106.5 64.5) (width 0.2) (layer "B.Cu") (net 37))
 (segment (start 113 65) (end 113 68.54) (width 0.2) (layer "B.Cu") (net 37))
 (segment (start 106.4 69.5) (end 106.4 64.6) (width 0.2) (layer "B.Cu") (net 37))
 (segment (start 112.5 64.5) (end 113 65) (width 0.2) (layer "B.Cu") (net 37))
 (segment (start 106.5 64.5) (end 112.5 64.5) (width 0.2) (layer "B.Cu") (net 37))
 (segment (start 113 74) (end 113.5 73.5) (width 0.2) (layer "B.Cu") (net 10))
 (segment (start 113.5 73.5) (end 113.5 76.765) (width 0.2) (layer "B.Cu") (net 10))
 (segment (start 106.5 74) (end 113 74) (width 0.2) (layer "B.Cu") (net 10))
 (segment (start 113.5 76.765) (end 112.265 78) (width 0.2) (layer "B.Cu") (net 10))
 (segment (start 106.5 78) (end 106.5 74) (width 0.2) (layer "B.Cu") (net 10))
 (segment (start 108 82.5) (end 113 82.5) (width 0.2) (layer "B.Cu") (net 2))
 (segment (start 106.9 87) (end 106.9 83.6) (width 0.2) (layer "B.Cu") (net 2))
 (segment (start 113 82.5) (end 112.265 83.235) (width 0.2) (layer "B.Cu") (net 2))
 (segment (start 112.265 83.235) (end 112.265 87) (width 0.2) (layer "B.Cu") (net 2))
 (segment (start 106.9 83.6) (end 108 82.5) (width 0.2) (layer "B.Cu") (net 2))
 (segment (start 94.1 201.6) (end 91 201.6) (width 0.2) (layer "F.Cu") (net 9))
 (segment (start 99.5 207) (end 94.1 201.6) (width 0.2) (layer "F.Cu") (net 9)))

